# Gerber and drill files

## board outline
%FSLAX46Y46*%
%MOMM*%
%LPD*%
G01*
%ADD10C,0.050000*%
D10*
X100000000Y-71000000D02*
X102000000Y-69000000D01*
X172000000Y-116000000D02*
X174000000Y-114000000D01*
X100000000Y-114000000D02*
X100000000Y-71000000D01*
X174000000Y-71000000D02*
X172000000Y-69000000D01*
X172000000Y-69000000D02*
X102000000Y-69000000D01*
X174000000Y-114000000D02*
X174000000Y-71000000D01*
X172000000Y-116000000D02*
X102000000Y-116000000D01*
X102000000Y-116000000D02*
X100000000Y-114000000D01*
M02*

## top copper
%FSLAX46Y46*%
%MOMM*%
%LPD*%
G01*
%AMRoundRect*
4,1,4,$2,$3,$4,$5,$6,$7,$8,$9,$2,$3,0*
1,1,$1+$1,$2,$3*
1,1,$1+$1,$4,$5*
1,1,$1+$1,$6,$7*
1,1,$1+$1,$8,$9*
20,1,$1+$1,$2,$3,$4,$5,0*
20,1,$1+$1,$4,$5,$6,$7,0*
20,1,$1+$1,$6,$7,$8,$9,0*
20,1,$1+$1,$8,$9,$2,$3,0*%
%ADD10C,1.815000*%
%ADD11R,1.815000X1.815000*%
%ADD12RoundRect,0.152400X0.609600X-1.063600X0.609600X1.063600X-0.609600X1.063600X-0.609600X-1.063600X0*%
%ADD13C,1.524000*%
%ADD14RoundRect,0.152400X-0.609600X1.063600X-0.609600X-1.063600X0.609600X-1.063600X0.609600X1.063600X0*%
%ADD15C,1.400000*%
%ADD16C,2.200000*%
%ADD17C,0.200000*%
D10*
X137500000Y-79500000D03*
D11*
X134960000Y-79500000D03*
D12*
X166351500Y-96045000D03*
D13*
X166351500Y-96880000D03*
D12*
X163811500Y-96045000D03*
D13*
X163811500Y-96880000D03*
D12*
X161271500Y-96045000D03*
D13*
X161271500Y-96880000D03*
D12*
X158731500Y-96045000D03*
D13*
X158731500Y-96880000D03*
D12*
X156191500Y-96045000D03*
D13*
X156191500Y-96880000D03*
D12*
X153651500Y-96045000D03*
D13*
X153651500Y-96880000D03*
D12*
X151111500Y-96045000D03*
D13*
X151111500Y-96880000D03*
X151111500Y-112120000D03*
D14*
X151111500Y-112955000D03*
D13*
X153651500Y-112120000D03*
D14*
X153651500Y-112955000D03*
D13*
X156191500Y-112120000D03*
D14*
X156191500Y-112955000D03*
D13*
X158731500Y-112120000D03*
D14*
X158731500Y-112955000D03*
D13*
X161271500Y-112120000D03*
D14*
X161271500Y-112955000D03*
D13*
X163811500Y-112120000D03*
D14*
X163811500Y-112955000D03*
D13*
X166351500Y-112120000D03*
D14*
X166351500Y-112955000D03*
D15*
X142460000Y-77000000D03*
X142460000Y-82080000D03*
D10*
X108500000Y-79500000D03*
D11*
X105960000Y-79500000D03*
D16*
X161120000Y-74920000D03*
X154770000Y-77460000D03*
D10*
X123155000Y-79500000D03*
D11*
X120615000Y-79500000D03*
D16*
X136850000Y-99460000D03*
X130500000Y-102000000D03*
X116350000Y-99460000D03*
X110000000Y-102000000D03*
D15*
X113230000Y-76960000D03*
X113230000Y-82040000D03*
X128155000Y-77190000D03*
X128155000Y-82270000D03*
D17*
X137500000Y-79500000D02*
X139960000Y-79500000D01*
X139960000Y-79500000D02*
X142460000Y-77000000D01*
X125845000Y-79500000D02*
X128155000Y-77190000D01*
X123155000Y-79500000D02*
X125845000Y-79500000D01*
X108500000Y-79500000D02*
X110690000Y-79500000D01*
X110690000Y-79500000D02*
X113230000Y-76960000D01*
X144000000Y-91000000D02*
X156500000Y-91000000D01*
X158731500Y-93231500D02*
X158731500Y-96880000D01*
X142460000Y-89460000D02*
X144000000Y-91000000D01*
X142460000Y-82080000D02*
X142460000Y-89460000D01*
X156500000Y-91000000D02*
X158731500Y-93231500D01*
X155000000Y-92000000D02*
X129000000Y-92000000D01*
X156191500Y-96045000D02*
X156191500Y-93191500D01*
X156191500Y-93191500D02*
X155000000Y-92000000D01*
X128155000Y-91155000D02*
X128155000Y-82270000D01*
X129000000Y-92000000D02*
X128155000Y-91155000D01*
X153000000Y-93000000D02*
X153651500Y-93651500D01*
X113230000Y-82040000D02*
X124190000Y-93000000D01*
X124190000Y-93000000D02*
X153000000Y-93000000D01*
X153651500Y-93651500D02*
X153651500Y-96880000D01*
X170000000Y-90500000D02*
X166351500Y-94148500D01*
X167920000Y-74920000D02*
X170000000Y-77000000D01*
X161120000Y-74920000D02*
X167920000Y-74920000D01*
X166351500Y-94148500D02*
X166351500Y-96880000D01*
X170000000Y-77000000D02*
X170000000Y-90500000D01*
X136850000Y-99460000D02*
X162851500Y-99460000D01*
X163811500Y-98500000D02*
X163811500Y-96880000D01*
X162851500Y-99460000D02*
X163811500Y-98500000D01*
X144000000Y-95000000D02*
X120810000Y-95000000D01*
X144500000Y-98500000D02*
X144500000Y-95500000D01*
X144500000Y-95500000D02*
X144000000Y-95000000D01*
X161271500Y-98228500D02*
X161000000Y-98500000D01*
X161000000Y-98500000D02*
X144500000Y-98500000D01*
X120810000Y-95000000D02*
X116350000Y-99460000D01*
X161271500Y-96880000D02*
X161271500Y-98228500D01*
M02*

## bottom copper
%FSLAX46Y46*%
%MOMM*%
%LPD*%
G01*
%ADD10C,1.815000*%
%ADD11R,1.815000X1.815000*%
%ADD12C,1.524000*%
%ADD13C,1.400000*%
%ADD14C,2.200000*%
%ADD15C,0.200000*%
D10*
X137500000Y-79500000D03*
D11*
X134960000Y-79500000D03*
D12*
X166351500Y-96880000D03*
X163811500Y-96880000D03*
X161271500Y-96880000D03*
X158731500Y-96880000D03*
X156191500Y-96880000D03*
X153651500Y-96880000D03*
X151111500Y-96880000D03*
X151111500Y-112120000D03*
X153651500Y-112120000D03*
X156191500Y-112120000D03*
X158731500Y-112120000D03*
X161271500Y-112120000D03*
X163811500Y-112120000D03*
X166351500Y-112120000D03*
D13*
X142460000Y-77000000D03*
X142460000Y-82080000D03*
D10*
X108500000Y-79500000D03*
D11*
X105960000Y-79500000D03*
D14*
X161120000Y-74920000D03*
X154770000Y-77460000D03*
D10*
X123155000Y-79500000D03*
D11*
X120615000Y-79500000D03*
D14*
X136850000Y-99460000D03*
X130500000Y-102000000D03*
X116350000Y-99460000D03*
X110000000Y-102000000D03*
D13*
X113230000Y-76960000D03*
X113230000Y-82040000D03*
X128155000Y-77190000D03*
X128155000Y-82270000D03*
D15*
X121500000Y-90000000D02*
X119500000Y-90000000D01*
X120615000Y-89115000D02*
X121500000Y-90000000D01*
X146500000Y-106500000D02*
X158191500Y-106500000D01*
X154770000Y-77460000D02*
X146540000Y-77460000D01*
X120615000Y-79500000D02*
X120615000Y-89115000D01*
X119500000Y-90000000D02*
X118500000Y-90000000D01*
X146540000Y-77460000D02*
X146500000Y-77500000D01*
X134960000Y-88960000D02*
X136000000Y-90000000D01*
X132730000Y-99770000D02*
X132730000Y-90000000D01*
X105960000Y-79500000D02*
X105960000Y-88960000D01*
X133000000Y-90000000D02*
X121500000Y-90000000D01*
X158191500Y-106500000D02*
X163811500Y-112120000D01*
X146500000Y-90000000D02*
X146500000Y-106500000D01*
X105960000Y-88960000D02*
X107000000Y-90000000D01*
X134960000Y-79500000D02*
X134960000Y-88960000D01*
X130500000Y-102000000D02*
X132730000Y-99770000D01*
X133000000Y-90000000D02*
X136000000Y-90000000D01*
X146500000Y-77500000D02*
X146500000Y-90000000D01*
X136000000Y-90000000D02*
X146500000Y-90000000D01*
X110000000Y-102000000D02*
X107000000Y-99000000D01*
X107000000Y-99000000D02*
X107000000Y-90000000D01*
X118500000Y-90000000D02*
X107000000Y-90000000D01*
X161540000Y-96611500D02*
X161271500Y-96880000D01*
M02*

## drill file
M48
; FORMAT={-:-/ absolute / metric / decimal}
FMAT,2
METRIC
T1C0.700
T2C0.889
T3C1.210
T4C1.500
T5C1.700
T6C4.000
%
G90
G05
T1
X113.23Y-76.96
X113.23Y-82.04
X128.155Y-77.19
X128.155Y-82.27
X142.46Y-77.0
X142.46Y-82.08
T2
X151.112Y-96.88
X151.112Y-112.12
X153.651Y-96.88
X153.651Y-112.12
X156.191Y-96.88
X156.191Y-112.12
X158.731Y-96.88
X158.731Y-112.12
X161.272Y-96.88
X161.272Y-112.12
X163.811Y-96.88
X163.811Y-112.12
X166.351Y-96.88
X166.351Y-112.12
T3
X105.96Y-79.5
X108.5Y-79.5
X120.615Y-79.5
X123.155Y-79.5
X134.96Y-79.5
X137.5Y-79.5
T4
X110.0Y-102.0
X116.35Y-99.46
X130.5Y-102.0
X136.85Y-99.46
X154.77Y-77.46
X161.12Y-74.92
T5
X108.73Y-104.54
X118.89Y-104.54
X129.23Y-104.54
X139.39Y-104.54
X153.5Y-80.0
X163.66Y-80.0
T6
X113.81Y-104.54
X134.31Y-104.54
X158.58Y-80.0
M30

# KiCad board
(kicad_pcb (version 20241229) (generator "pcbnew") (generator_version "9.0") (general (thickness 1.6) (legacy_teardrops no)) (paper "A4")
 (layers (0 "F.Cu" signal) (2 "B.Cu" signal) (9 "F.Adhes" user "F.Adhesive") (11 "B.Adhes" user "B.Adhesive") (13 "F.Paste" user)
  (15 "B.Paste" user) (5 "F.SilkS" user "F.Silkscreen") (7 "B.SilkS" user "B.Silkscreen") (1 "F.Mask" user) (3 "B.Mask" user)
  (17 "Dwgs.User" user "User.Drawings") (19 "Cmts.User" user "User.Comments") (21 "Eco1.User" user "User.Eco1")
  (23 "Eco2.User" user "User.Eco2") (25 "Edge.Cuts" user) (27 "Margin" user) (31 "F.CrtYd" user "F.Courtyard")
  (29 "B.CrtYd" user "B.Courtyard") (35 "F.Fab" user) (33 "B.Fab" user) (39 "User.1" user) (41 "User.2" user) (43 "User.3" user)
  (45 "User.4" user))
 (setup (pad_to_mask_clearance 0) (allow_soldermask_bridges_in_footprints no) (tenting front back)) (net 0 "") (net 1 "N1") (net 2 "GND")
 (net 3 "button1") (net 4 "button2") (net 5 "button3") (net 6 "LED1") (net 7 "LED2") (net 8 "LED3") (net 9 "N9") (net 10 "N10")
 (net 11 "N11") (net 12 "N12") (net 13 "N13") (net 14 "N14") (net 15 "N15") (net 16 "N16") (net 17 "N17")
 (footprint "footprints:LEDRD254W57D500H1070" (layer "F.Cu") (at 136.23 79.5)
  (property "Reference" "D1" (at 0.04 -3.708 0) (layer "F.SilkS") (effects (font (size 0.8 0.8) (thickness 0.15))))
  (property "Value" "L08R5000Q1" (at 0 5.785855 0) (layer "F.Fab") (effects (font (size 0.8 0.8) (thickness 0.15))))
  (pad "A" thru_hole circle (at 1.27 0) (size 1.815 1.815) (drill 1.21) (layers "*.Cu" "*.Mask") (remove_unused_layers no) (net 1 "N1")
   (solder_mask_margin 0.102))
  (pad "C" thru_hole rect (at -1.27 0) (size 1.815 1.815) (drill 1.21) (layers "*.Cu" "*.Mask") (remove_unused_layers no) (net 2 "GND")
   (solder_mask_margin 0.102)))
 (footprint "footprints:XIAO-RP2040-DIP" (layer "F.Cu") (at 158.7315 104.5 -90)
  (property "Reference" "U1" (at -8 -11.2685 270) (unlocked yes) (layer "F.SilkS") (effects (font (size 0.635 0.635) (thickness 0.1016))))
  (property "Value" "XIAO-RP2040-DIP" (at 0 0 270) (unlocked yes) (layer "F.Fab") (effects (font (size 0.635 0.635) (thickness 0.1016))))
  (pad "1" smd roundrect (at -8.455 -7.62 90) (size 2.432 1.524) (layers "F.Cu" "F.Mask") (roundrect_rratio 0.1) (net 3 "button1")
   (thermal_bridge_angle 45))
  (pad "1" thru_hole circle (at -7.62 -7.62 90) (size 1.524 1.524) (drill 0.889) (layers "*.Cu" "*.Mask") (remove_unused_layers no)
   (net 3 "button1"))
  (pad "2" smd roundrect (at -8.455 -5.08 90) (size 2.432 1.524) (layers "F.Cu" "F.Mask") (roundrect_rratio 0.1) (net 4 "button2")
   (thermal_bridge_angle 45))
  (pad "2" thru_hole circle (at -7.62 -5.08 90) (size 1.524 1.524) (drill 0.889) (layers "*.Cu" "*.Mask") (remove_unused_layers no)
   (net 4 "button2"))
  (pad "3" smd roundrect (at -8.455 -2.54 90) (size 2.432 1.524) (layers "F.Cu" "F.Mask") (roundrect_rratio 0.1) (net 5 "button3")
   (thermal_bridge_angle 45))
  (pad "3" thru_hole circle (at -7.62 -2.54 90) (size 1.524 1.524) (drill 0.889) (layers "*.Cu" "*.Mask") (remove_unused_layers no)
   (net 5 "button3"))
  (pad "4" smd roundrect (at -8.455 0 90) (size 2.432 1.524) (layers "F.Cu" "F.Mask") (roundrect_rratio 0.1) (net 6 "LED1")
   (thermal_bridge_angle 45))
  (pad "4" thru_hole circle (at -7.62 0 90) (size 1.524 1.524) (drill 0.889) (layers "*.Cu" "*.Mask") (remove_unused_layers no)
   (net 6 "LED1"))
  (pad "5" smd roundrect (at -8.455 2.54 90) (size 2.432 1.524) (layers "F.Cu" "F.Mask") (roundrect_rratio 0.1) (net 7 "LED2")
   (thermal_bridge_angle 45))
  (pad "5" thru_hole circle (at -7.62 2.54 90) (size 1.524 1.524) (drill 0.889) (layers "*.Cu" "*.Mask") (remove_unused_layers no)
   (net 7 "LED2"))
  (pad "6" smd roundrect (at -8.455 5.08 90) (size 2.432 1.524) (layers "F.Cu" "F.Mask") (roundrect_rratio 0.1) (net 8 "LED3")
   (thermal_bridge_angle 45))
  (pad "6" thru_hole circle (at -7.62 5.08 90) (size 1.524 1.524) (drill 0.889) (layers "*.Cu" "*.Mask") (remove_unused_layers no)
   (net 8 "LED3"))
  (pad "7" smd roundrect (at -8.455 7.62 90) (size 2.432 1.524) (layers "F.Cu" "F.Mask") (roundrect_rratio 0.1) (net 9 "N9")
   (thermal_bridge_angle 45))
  (pad "7" thru_hole circle (at -7.62 7.62 90) (size 1.524 1.524) (drill 0.889) (layers "*.Cu" "*.Mask") (remove_unused_layers no)
   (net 9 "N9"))
  (pad "8" thru_hole circle (at 7.62 7.62 270) (size 1.524 1.524) (drill 0.889) (layers "*.Cu" "*.Mask") (remove_unused_layers no)
   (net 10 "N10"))
  (pad "8" smd roundrect (at 8.455 7.62 270) (size 2.432 1.524) (layers "F.Cu" "F.Mask") (roundrect_rratio 0.1) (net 10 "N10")
   (thermal_bridge_angle 45))
  (pad "9" thru_hole circle (at 7.62 5.08 270) (size 1.524 1.524) (drill 0.889) (layers "*.Cu" "*.Mask") (remove_unused_layers no)
   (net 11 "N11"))
  (pad "9" smd roundrect (at 8.455 5.08 270) (size 2.432 1.524) (layers "F.Cu" "F.Mask") (roundrect_rratio 0.1) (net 11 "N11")
   (thermal_bridge_angle 45))
  (pad "10" thru_hole circle (at 7.62 2.54 270) (size 1.524 1.524) (drill 0.889) (layers "*.Cu" "*.Mask") (remove_unused_layers no)
   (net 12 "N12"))
  (pad "10" smd roundrect (at 8.455 2.54 270) (size 2.432 1.524) (layers "F.Cu" "F.Mask") (roundrect_rratio 0.1) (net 12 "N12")
   (thermal_bridge_angle 45))
  (pad "11" thru_hole circle (at 7.62 0 270) (size 1.524 1.524) (drill 0.889) (layers "*.Cu" "*.Mask") (remove_unused_layers no)
   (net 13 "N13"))
  (pad "11" smd roundrect (at 8.455 0 270) (size 2.432 1.524) (layers "F.Cu" "F.Mask") (roundrect_rratio 0.1) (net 13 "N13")
   (thermal_bridge_angle 45))
  (pad "12" thru_hole circle (at 7.62 -2.54 270) (size 1.524 1.524) (drill 0.889) (layers "*.Cu" "*.Mask") (remove_unused_layers no)
   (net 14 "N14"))
  (pad "12" smd roundrect (at 8.455 -2.54 270) (size 2.432 1.524) (layers "F.Cu" "F.Mask") (roundrect_rratio 0.1) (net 14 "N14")
   (thermal_bridge_angle 45))
  (pad "13" thru_hole circle (at 7.62 -5.08 270) (size 1.524 1.524) (drill 0.889) (layers "*.Cu" "*.Mask") (remove_unused_layers no)
   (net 2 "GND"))
  (pad "13" smd roundrect (at 8.455 -5.08 270) (size 2.432 1.524) (layers "F.Cu" "F.Mask") (roundrect_rratio 0.1) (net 2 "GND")
   (thermal_bridge_angle 45))
  (pad "14" thru_hole circle (at 7.62 -7.62 270) (size 1.524 1.524) (drill 0.889) (layers "*.Cu" "*.Mask") (remove_unused_layers no)
   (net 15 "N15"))
  (pad "14" smd roundrect (at 8.455 -7.62 270) (size 2.432 1.524) (layers "F.Cu" "F.Mask") (roundrect_rratio 0.1) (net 15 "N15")
   (thermal_bridge_angle 45)))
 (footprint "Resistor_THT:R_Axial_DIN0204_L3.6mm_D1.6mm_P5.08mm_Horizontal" (layer "F.Cu") (at 142.46 77 -90)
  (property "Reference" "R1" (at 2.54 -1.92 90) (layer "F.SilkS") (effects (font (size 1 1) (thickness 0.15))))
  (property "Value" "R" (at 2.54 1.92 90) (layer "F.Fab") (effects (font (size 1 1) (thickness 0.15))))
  (pad "1" thru_hole circle (at 0 0 270) (size 1.4 1.4) (drill 0.7) (layers "*.Cu" "*.Mask") (remove_unused_layers no) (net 1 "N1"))
  (pad "2" thru_hole circle (at 5.08 0 270) (size 1.4 1.4) (drill 0.7) (layers "*.Cu" "*.Mask") (remove_unused_layers no) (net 6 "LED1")))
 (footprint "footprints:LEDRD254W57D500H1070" (layer "F.Cu") (at 107.23 79.5)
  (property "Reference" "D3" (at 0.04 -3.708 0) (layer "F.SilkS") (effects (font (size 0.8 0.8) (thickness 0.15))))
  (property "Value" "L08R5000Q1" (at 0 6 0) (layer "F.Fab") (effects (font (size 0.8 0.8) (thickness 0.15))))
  (pad "A" thru_hole circle (at 1.27 0) (size 1.815 1.815) (drill 1.21) (layers "*.Cu" "*.Mask") (remove_unused_layers no) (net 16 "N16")
   (solder_mask_margin 0.102))
  (pad "C" thru_hole rect (at -1.27 0) (size 1.815 1.815) (drill 1.21) (layers "*.Cu" "*.Mask") (remove_unused_layers no) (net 2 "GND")
   (solder_mask_margin 0.102)))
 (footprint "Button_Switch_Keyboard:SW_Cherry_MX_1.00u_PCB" (layer "F.Cu") (at 161.12 74.92)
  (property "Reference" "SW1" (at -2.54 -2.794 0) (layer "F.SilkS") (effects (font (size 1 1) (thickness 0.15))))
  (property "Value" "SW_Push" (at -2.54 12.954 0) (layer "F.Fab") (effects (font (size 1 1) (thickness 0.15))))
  (pad "" np_thru_hole circle (at -7.62 5.08) (size 1.7 1.7) (drill 1.7) (layers "*.Cu" "*.Mask"))
  (pad "" np_thru_hole circle (at -2.54 5.08) (size 4 4) (drill 4) (layers "*.Cu" "*.Mask"))
  (pad "" np_thru_hole circle (at 2.54 5.08) (size 1.7 1.7) (drill 1.7) (layers "*.Cu" "*.Mask"))
  (pad "1" thru_hole circle (at 0 0) (size 2.2 2.2) (drill 1.5) (layers "*.Cu" "*.Mask") (remove_unused_layers no) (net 3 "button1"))
  (pad "2" thru_hole circle (at -6.35 2.54) (size 2.2 2.2) (drill 1.5) (layers "*.Cu" "*.Mask") (remove_unused_layers no) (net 2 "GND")))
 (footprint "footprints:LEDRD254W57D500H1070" (layer "F.Cu") (at 121.885 79.5)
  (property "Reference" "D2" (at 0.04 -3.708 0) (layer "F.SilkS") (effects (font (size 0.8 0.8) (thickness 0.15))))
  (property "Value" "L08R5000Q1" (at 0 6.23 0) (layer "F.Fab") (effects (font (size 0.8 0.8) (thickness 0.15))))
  (pad "A" thru_hole circle (at 1.27 0) (size 1.815 1.815) (drill 1.21) (layers "*.Cu" "*.Mask") (remove_unused_layers no) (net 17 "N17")
   (solder_mask_margin 0.102))
  (pad "C" thru_hole rect (at -1.27 0) (size 1.815 1.815) (drill 1.21) (layers "*.Cu" "*.Mask") (remove_unused_layers no) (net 2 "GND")
   (solder_mask_margin 0.102)))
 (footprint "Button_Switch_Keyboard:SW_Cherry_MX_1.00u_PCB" (layer "F.Cu") (at 136.85 99.46)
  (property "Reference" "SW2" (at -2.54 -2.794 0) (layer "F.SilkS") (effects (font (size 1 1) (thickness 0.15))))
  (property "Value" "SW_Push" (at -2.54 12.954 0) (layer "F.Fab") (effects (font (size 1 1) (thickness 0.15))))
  (pad "" np_thru_hole circle (at -7.62 5.08) (size 1.7 1.7) (drill 1.7) (layers "*.Cu" "*.Mask"))
  (pad "" np_thru_hole circle (at -2.54 5.08) (size 4 4) (drill 4) (layers "*.Cu" "*.Mask"))
  (pad "" np_thru_hole circle (at 2.54 5.08) (size 1.7 1.7) (drill 1.7) (layers "*.Cu" "*.Mask"))
  (pad "1" thru_hole circle (at 0 0) (size 2.2 2.2) (drill 1.5) (layers "*.Cu" "*.Mask") (remove_unused_layers no) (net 4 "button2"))
  (pad "2" thru_hole circle (at -6.35 2.54) (size 2.2 2.2) (drill 1.5) (layers "*.Cu" "*.Mask") (remove_unused_layers no) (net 2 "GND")))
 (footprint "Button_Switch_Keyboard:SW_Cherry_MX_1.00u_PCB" (layer "F.Cu") (at 116.35 99.46)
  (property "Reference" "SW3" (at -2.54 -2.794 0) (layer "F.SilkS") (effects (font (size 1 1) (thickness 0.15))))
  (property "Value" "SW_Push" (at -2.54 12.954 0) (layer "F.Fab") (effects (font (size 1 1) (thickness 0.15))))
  (pad "" np_thru_hole circle (at -7.62 5.08) (size 1.7 1.7) (drill 1.7) (layers "*.Cu" "*.Mask"))
  (pad "" np_thru_hole circle (at -2.54 5.08) (size 4 4) (drill 4) (layers "*.Cu" "*.Mask"))
  (pad "" np_thru_hole circle (at 2.54 5.08) (size 1.7 1.7) (drill 1.7) (layers "*.Cu" "*.Mask"))
  (pad "1" thru_hole circle (at 0 0) (size 2.2 2.2) (drill 1.5) (layers "*.Cu" "*.Mask") (remove_unused_layers no) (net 5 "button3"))
  (pad "2" thru_hole circle (at -6.35 2.54) (size 2.2 2.2) (drill 1.5) (layers "*.Cu" "*.Mask") (remove_unused_layers no) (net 2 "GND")))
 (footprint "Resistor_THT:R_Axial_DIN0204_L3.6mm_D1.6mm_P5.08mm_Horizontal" (layer "F.Cu") (at 113.23 76.96 -90)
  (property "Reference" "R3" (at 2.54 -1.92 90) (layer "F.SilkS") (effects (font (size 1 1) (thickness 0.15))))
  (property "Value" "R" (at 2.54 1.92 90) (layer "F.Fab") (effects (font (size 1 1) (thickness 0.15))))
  (pad "1" thru_hole circle (at 0 0 270) (size 1.4 1.4) (drill 0.7) (layers "*.Cu" "*.Mask") (remove_unused_layers no) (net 16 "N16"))
  (pad "2" thru_hole circle (at 5.08 0 270) (size 1.4 1.4) (drill 0.7) (layers "*.Cu" "*.Mask") (remove_unused_layers no) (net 8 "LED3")))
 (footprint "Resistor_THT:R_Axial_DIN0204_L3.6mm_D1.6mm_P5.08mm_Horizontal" (layer "F.Cu") (at 128.155 77.19 -90)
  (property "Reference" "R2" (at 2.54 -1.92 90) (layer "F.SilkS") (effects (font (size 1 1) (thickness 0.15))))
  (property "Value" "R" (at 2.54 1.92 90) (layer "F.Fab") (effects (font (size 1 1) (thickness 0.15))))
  (pad "1" thru_hole circle (at 0 0 270) (size 1.4 1.4) (drill 0.7) (layers "*.Cu" "*.Mask") (remove_unused_layers no) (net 17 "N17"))
  (pad "2" thru_hole circle (at 5.08 0 270) (size 1.4 1.4) (drill 0.7) (layers "*.Cu" "*.Mask") (remove_unused_layers no) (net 7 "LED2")))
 (gr_line (start 100 71) (end 102 69) (stroke (width 0.05) (type default)) (layer "Edge.Cuts"))
 (gr_line (start 172 116) (end 174 114) (stroke (width 0.05) (type default)) (layer "Edge.Cuts"))
 (gr_line (start 100 114) (end 100 71) (stroke (width 0.05) (type default)) (layer "Edge.Cuts"))
 (gr_line (start 174 71) (end 172 69) (stroke (width 0.05) (type default)) (layer "Edge.Cuts"))
 (gr_line (start 172 69) (end 102 69) (stroke (width 0.05) (type default)) (layer "Edge.Cuts"))
 (gr_line (start 174 114) (end 174 71) (stroke (width 0.05) (type default)) (layer "Edge.Cuts"))
 (gr_line (start 172 116) (end 102 116) (stroke (width 0.05) (type default)) (layer "Edge.Cuts"))
 (gr_line (start 102 116) (end 100 114) (stroke (width 0.05) (type default)) (layer "Edge.Cuts"))
 (segment (start 121.5 90) (end 119.5 90) (width 0.2) (layer "B.Cu") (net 2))
 (segment (start 120.615 89.115) (end 121.5 90) (width 0.2) (layer "B.Cu") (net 2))
 (segment (start 146.5 106.5) (end 158.1915 106.5) (width 0.2) (layer "B.Cu") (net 2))
 (segment (start 154.77 77.46) (end 146.54 77.46) (width 0.2) (layer "B.Cu") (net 2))
 (segment (start 120.615 79.5) (end 120.615 89.115) (width 0.2) (layer "B.Cu") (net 2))
 (segment (start 119.5 90) (end 118.5 90) (width 0.2) (layer "B.Cu") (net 2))
 (segment (start 146.54 77.46) (end 146.5 77.5) (width 0.2) (layer "B.Cu") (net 2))
 (segment (start 134.96 88.96) (end 136 90) (width 0.2) (layer "B.Cu") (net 2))
 (segment (start 132.73 99.77) (end 132.73 90) (width 0.2) (layer "B.Cu") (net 2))
 (segment (start 105.96 79.5) (end 105.96 88.96) (width 0.2) (layer "B.Cu") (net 2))
 (segment (start 133 90) (end 121.5 90) (width 0.2) (layer "B.Cu") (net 2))
 (segment (start 158.1915 106.5) (end 163.8115 112.12) (width 0.2) (layer "B.Cu") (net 2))
 (segment (start 146.5 90) (end 146.5 106.5) (width 0.2) (layer "B.Cu") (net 2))
 (segment (start 105.96 88.96) (end 107 90) (width 0.2) (layer "B.Cu") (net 2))
 (segment (start 134.96 79.5) (end 134.96 88.96) (width 0.2) (layer "B.Cu") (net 2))
 (segment (start 130.5 102) (end 132.73 99.77) (width 0.2) (layer "B.Cu") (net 2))
 (segment (start 133 90) (end 136 90) (width 0.2) (layer "B.Cu") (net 2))
 (segment (start 146.5 77.5) (end 146.5 90) (width 0.2) (layer "B.Cu") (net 2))
 (segment (start 136 90) (end 146.5 90) (width 0.2) (layer "B.Cu") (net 2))
 (segment (start 110 102) (end 107 99) (width 0.2) (layer "B.Cu") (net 2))
 (segment (start 107 99) (end 107 90) (width 0.2) (layer "B.Cu") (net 2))
 (segment (start 118.5 90) (end 107 90) (width 0.2) (layer "B.Cu") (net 2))
 (segment (start 137.5 79.5) (end 139.96 79.5) (width 0.2) (layer "F.Cu") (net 1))
 (segment (start 139.96 79.5) (end 142.46 77) (width 0.2) (layer "F.Cu") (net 1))
 (segment (start 125.845 79.5) (end 128.155 77.19) (width 0.2) (layer "F.Cu") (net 17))
 (segment (start 123.155 79.5) (end 125.845 79.5) (width 0.2) (layer "F.Cu") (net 17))
 (segment (start 108.5 79.5) (end 110.69 79.5) (width 0.2) (layer "F.Cu") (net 16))
 (segment (start 110.69 79.5) (end 113.23 76.96) (width 0.2) (layer "F.Cu") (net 16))
 (segment (start 144 91) (end 156.5 91) (width 0.2) (layer "F.Cu") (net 6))
 (segment (start 158.7315 93.2315) (end 158.7315 96.88) (width 0.2) (layer "F.Cu") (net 6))
 (segment (start 142.46 89.46) (end 144 91) (width 0.2) (layer "F.Cu") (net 6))
 (segment (start 142.46 82.08) (end 142.46 89.46) (width 0.2) (layer "F.Cu") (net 6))
 (segment (start 156.5 91) (end 158.7315 93.2315) (width 0.2) (layer "F.Cu") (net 6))
 (segment (start 155 92) (end 129 92) (width 0.2) (layer "F.Cu") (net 7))
 (segment (start 156.1915 96.045) (end 156.1915 93.1915) (width 0.2) (layer "F.Cu") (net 7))
 (segment (start 156.1915 93.1915) (end 155 92) (width 0.2) (layer "F.Cu") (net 7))
 (segment (start 128.155 91.155) (end 128.155 82.27) (width 0.2) (layer "F.Cu") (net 7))
 (segment (start 129 92) (end 128.155 91.155) (width 0.2) (layer "F.Cu") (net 7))
 (segment (start 153 93) (end 153.6515 93.6515) (width 0.2) (layer "F.Cu") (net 8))
 (segment (start 113.23 82.04) (end 124.19 93) (width 0.2) (layer "F.Cu") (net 8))
 (segment (start 124.19 93) (end 153 93) (width 0.2) (layer "F.Cu") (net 8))
 (segment (start 153.6515 93.6515) (end 153.6515 96.88) (width 0.2) (layer "F.Cu") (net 8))
 (segment (start 170 90.5) (end 166.3515 94.1485) (width 0.2) (layer "F.Cu") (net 3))
 (segment (start 167.92 74.92) (end 170 77) (width 0.2) (layer "F.Cu") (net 3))
 (segment (start 161.12 74.92) (end 167.92 74.92) (width 0.2) (layer "F.Cu") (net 3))
 (segment (start 166.3515 94.1485) (end 166.3515 96.88) (width 0.2) (layer "F.Cu") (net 3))
 (segment (start 170 77) (end 170 90.5) (width 0.2) (layer "F.Cu") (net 3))
 (segment (start 136.85 99.46) (end 162.8515 99.46) (width 0.2) (layer "F.Cu") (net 4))
 (segment (start 163.8115 98.5) (end 163.8115 96.88) (width 0.2) (layer "F.Cu") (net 4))
 (segment (start 162.8515 99.46) (end 163.8115 98.5) (width 0.2) (layer "F.Cu") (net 4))
 (segment (start 144 95) (end 120.81 95) (width 0.2) (layer "F.Cu") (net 5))
 (segment (start 144.5 98.5) (end 144.5 95.5) (width 0.2) (layer "F.Cu") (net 5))
 (segment (start 144.5 95.5) (end 144 95) (width 0.2) (layer "F.Cu") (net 5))
 (segment (start 161.2715 98.2285) (end 161 98.5) (width 0.2) (layer "F.Cu") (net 5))
 (segment (start 161 98.5) (end 144.5 98.5) (width 0.2) (layer "F.Cu") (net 5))
 (segment (start 120.81 95) (end 116.35 99.46) (width 0.2) (layer "F.Cu") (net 5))
 (segment (start 161.2715 96.88) (end 161.2715 98.2285) (width 0.2) (layer "F.Cu") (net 5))
 (segment (start 161.54 96.6115) (end 161.2715 96.88) (width 0.2) (layer "B.Cu") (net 5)))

